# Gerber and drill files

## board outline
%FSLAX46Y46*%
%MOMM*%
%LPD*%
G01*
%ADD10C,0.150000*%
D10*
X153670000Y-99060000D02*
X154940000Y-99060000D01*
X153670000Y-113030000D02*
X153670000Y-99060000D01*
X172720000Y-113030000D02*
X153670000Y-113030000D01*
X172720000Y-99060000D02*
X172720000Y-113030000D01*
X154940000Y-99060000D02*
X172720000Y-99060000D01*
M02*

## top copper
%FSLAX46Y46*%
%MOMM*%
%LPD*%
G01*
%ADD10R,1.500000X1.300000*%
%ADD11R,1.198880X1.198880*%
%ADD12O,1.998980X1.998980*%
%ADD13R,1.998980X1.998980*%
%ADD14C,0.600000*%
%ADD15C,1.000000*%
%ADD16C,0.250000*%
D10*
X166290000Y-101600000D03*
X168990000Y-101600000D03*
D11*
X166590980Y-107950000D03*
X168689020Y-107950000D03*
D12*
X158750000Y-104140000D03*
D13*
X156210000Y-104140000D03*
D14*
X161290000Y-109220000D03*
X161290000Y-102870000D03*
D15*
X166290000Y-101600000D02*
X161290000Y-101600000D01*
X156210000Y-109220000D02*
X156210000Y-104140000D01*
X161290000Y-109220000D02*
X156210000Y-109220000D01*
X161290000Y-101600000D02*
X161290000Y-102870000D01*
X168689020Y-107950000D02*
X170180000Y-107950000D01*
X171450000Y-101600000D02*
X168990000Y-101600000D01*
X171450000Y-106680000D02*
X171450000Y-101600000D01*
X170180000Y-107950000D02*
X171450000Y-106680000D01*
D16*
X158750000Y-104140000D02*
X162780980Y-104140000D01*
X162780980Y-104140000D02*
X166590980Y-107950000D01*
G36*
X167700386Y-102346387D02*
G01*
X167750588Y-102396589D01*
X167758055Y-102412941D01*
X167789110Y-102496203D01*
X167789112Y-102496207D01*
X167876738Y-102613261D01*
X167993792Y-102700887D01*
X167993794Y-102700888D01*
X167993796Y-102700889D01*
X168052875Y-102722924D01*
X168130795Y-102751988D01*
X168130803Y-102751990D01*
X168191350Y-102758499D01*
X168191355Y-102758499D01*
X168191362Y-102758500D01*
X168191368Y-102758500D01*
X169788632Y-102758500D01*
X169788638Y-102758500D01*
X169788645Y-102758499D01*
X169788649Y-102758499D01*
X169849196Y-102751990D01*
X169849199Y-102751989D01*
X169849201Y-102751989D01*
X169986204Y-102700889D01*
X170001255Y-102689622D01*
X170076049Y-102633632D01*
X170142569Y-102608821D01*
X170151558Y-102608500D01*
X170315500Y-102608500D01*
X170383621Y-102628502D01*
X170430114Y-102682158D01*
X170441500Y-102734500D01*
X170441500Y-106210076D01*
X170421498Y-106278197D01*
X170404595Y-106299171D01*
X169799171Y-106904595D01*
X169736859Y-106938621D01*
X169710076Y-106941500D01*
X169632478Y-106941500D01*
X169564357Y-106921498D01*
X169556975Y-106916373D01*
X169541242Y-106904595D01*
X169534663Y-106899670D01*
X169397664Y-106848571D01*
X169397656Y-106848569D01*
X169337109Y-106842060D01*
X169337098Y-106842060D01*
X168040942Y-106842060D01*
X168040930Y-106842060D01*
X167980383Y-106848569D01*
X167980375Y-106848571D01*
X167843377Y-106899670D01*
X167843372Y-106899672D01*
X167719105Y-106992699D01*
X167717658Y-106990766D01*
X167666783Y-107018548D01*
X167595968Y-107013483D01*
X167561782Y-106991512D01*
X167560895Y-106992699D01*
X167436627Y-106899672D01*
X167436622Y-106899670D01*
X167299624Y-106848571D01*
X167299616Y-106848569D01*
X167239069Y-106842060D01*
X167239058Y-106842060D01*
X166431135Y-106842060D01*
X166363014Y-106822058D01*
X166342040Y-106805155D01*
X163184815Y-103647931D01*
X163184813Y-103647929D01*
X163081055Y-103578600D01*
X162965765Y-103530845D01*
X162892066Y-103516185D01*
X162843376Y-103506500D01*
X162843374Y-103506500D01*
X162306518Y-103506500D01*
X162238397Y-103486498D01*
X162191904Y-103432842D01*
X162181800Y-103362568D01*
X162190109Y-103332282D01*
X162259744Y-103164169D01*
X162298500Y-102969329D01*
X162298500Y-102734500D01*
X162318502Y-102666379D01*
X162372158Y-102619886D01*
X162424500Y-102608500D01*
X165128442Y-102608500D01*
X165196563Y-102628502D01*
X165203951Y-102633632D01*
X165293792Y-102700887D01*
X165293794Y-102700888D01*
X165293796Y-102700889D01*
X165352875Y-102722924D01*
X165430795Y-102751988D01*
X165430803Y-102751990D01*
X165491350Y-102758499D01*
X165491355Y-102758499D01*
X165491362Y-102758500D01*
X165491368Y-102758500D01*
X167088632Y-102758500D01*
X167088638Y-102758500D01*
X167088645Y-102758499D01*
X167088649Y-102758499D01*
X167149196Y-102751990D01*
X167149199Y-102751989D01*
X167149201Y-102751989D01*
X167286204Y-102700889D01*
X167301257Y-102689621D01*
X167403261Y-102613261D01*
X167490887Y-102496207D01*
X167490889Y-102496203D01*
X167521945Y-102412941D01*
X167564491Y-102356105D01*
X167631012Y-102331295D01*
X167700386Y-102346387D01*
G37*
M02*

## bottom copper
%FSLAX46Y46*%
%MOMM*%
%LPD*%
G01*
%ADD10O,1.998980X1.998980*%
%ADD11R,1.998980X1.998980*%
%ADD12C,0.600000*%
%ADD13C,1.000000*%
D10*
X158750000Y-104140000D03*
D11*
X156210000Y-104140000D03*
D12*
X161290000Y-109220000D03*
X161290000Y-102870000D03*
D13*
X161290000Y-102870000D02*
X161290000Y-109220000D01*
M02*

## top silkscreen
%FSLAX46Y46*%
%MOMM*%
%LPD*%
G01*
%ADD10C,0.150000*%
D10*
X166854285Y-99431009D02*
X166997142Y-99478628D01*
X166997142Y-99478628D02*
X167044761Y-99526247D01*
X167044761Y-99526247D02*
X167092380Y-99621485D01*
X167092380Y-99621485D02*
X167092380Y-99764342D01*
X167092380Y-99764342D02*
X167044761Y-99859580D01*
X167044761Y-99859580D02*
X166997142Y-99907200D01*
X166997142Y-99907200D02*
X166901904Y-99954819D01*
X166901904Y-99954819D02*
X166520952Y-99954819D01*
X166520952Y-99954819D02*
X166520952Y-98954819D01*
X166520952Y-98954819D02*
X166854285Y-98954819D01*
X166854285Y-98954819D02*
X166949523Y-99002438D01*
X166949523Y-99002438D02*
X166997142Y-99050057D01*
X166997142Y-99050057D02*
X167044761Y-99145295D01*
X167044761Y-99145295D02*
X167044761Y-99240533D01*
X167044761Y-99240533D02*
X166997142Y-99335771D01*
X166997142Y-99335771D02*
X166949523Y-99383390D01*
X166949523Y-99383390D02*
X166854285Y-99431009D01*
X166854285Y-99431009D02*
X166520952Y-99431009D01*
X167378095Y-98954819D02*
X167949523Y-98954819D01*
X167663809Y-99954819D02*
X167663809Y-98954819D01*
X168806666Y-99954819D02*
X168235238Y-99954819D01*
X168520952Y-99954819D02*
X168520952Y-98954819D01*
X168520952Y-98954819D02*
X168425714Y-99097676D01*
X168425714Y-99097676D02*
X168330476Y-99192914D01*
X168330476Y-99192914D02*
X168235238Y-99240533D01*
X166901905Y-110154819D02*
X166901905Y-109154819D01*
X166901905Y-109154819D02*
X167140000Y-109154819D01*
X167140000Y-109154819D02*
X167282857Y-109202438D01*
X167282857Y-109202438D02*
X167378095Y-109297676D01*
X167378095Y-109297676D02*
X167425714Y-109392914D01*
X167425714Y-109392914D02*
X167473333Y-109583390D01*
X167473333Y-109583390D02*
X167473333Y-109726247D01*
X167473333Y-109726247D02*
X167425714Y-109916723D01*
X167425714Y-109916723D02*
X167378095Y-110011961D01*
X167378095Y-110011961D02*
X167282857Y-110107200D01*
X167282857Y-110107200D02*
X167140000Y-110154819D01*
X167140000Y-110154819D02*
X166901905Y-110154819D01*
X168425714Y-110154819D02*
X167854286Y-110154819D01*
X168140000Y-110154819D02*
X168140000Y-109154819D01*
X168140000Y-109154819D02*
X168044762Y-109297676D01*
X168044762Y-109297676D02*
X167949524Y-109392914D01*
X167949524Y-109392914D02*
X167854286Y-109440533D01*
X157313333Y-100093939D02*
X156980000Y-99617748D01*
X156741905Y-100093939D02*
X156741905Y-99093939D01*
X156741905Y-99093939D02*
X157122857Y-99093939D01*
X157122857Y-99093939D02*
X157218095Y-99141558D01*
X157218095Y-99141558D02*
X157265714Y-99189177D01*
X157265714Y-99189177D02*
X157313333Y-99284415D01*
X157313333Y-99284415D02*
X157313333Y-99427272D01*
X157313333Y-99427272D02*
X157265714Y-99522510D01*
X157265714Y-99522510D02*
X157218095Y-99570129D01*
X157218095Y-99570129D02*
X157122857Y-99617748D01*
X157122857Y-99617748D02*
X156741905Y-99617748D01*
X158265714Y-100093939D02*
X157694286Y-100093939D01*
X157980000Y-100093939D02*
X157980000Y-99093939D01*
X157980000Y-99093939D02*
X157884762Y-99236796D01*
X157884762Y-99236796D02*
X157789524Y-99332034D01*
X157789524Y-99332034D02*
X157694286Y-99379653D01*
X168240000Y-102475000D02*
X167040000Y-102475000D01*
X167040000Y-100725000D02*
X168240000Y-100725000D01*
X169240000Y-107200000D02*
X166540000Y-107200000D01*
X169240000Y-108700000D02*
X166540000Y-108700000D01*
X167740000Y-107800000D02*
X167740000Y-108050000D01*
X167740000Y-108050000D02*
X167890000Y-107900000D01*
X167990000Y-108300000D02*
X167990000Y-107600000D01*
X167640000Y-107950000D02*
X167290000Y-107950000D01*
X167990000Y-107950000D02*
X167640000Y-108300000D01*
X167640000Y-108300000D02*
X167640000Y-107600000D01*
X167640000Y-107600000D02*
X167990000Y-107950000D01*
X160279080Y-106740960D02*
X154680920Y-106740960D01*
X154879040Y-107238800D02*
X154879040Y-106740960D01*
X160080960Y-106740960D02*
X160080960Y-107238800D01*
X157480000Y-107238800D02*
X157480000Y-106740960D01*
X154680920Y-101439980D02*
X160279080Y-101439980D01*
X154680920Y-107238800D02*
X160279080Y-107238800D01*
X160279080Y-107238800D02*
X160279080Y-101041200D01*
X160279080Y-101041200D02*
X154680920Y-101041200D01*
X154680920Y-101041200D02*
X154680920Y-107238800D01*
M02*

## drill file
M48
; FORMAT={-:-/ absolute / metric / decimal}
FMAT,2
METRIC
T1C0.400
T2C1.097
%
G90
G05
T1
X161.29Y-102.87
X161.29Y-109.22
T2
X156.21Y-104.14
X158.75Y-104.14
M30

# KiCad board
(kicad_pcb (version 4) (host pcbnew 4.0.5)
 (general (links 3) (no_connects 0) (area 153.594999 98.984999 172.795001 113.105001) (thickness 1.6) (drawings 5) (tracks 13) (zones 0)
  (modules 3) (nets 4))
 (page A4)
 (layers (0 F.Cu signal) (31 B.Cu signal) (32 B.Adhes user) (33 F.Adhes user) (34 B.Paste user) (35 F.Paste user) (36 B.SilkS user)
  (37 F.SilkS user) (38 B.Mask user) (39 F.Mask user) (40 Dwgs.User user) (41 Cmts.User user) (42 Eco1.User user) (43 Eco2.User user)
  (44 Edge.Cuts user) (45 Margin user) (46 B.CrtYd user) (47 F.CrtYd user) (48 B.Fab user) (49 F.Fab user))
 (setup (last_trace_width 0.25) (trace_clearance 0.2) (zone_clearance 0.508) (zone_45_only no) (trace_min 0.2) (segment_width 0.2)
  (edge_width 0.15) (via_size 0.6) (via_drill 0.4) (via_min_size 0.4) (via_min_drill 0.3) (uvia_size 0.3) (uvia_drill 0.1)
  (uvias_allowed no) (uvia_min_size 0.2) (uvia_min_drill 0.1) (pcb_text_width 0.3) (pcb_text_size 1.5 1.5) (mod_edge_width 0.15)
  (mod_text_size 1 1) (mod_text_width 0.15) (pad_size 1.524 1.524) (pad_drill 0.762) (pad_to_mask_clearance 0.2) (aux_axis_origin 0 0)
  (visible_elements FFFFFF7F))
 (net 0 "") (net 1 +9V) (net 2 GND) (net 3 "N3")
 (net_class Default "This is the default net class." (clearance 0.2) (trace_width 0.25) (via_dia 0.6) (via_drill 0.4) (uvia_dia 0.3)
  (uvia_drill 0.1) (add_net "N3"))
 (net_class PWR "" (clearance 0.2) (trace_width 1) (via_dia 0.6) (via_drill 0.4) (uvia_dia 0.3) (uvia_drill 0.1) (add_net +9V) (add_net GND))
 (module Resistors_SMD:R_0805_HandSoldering (layer F.Cu) (at 167.64 101.6)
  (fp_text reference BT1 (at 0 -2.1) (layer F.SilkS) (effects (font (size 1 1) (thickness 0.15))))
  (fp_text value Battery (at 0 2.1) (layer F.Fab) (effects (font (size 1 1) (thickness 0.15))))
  (fp_line (start 0.6 0.875) (end -0.6 0.875) (layer F.SilkS) (width 0.15))
  (fp_line (start -0.6 -0.875) (end 0.6 -0.875) (layer F.SilkS) (width 0.15))
  (pad 1 smd rect (at -1.35 0) (size 1.5 1.3) (layers F.Cu F.Paste F.Mask) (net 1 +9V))
  (pad 2 smd rect (at 1.35 0) (size 1.5 1.3) (layers F.Cu F.Paste F.Mask) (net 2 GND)))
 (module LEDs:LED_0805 (layer F.Cu) (at 167.64 107.95 180)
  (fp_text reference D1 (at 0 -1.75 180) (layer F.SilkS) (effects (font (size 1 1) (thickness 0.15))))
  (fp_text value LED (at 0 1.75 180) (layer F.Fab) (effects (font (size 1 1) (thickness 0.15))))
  (fp_line (start -1.6 0.75) (end 1.1 0.75) (layer F.SilkS) (width 0.15))
  (fp_line (start -1.6 -0.75) (end 1.1 -0.75) (layer F.SilkS) (width 0.15))
  (fp_line (start -0.1 0.15) (end -0.1 -0.1) (layer F.SilkS) (width 0.15))
  (fp_line (start -0.1 -0.1) (end -0.25 0.05) (layer F.SilkS) (width 0.15))
  (fp_line (start -0.35 -0.35) (end -0.35 0.35) (layer F.SilkS) (width 0.15))
  (fp_line (start 0 0) (end 0.35 0) (layer F.SilkS) (width 0.15))
  (fp_line (start -0.35 0) (end 0 -0.35) (layer F.SilkS) (width 0.15))
  (fp_line (start 0 -0.35) (end 0 0.35) (layer F.SilkS) (width 0.15))
  (fp_line (start 0 0.35) (end -0.35 0) (layer F.SilkS) (width 0.15))
  (pad 2 smd rect (at 1.04902 0) (size 1.19888 1.19888) (layers F.Cu F.Paste F.Mask) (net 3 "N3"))
  (pad 1 smd rect (at -1.04902 0) (size 1.19888 1.19888) (layers F.Cu F.Paste F.Mask) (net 2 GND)))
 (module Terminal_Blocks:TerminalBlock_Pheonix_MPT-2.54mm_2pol (layer F.Cu) (at 156.21 104.14)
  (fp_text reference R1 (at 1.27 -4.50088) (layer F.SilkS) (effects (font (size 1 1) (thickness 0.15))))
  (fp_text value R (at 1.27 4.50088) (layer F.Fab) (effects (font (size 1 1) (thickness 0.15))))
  (fp_line (start 4.06908 2.60096) (end -1.52908 2.60096) (layer F.SilkS) (width 0.15))
  (fp_line (start -1.33096 3.0988) (end -1.33096 2.60096) (layer F.SilkS) (width 0.15))
  (fp_line (start 3.87096 2.60096) (end 3.87096 3.0988) (layer F.SilkS) (width 0.15))
  (fp_line (start 1.27 3.0988) (end 1.27 2.60096) (layer F.SilkS) (width 0.15))
  (fp_line (start -1.52908 -2.70002) (end 4.06908 -2.70002) (layer F.SilkS) (width 0.15))
  (fp_line (start -1.52908 3.0988) (end 4.06908 3.0988) (layer F.SilkS) (width 0.15))
  (fp_line (start 4.06908 3.0988) (end 4.06908 -3.0988) (layer F.SilkS) (width 0.15))
  (fp_line (start 4.06908 -3.0988) (end -1.52908 -3.0988) (layer F.SilkS) (width 0.15))
  (fp_line (start -1.52908 -3.0988) (end -1.52908 3.0988) (layer F.SilkS) (width 0.15))
  (pad 2 thru_hole oval (at 2.54 0) (size 1.99898 1.99898) (drill 1.09728) (layers *.Cu *.Mask) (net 3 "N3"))
  (pad 1 thru_hole rect (at 0 0) (size 1.99898 1.99898) (drill 1.09728) (layers *.Cu *.Mask) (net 1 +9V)))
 (gr_line (start 153.67 99.06) (end 154.94 99.06) (angle 90) (layer Edge.Cuts) (width 0.15))
 (gr_line (start 153.67 113.03) (end 153.67 99.06) (angle 90) (layer Edge.Cuts) (width 0.15))
 (gr_line (start 172.72 113.03) (end 153.67 113.03) (angle 90) (layer Edge.Cuts) (width 0.15))
 (gr_line (start 172.72 99.06) (end 172.72 113.03) (angle 90) (layer Edge.Cuts) (width 0.15))
 (gr_line (start 154.94 99.06) (end 172.72 99.06) (angle 90) (layer Edge.Cuts) (width 0.15))
 (segment (start 166.29 101.6) (end 161.29 101.6) (width 1) (layer F.Cu) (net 1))
 (segment (start 156.21 109.22) (end 156.21 104.14) (width 1) (layer F.Cu) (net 1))
 (segment (start 161.29 109.22) (end 156.21 109.22) (width 1) (layer F.Cu) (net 1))
 (via (at 161.29 109.22) (size 0.6) (drill 0.4) (layers F.Cu B.Cu) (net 1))
 (segment (start 161.29 102.87) (end 161.29 109.22) (width 1) (layer B.Cu) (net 1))
 (via (at 161.29 102.87) (size 0.6) (drill 0.4) (layers F.Cu B.Cu) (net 1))
 (segment (start 161.29 101.6) (end 161.29 102.87) (width 1) (layer F.Cu) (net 1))
 (segment (start 168.68902 107.95) (end 170.18 107.95) (width 1) (layer F.Cu) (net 2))
 (segment (start 171.45 101.6) (end 168.99 101.6) (width 1) (layer F.Cu) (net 2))
 (segment (start 171.45 106.68) (end 171.45 101.6) (width 1) (layer F.Cu) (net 2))
 (segment (start 170.18 107.95) (end 171.45 106.68) (width 1) (layer F.Cu) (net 2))
 (segment (start 158.75 104.14) (end 162.78098 104.14) (width 0.25) (layer F.Cu) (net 3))
 (segment (start 162.78098 104.14) (end 166.59098 107.95) (width 0.25) (layer F.Cu) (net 3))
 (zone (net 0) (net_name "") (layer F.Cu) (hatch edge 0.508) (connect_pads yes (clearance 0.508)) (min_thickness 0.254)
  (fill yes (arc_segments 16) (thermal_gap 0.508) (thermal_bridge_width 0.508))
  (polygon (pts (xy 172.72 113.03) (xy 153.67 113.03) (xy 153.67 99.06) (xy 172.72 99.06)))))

